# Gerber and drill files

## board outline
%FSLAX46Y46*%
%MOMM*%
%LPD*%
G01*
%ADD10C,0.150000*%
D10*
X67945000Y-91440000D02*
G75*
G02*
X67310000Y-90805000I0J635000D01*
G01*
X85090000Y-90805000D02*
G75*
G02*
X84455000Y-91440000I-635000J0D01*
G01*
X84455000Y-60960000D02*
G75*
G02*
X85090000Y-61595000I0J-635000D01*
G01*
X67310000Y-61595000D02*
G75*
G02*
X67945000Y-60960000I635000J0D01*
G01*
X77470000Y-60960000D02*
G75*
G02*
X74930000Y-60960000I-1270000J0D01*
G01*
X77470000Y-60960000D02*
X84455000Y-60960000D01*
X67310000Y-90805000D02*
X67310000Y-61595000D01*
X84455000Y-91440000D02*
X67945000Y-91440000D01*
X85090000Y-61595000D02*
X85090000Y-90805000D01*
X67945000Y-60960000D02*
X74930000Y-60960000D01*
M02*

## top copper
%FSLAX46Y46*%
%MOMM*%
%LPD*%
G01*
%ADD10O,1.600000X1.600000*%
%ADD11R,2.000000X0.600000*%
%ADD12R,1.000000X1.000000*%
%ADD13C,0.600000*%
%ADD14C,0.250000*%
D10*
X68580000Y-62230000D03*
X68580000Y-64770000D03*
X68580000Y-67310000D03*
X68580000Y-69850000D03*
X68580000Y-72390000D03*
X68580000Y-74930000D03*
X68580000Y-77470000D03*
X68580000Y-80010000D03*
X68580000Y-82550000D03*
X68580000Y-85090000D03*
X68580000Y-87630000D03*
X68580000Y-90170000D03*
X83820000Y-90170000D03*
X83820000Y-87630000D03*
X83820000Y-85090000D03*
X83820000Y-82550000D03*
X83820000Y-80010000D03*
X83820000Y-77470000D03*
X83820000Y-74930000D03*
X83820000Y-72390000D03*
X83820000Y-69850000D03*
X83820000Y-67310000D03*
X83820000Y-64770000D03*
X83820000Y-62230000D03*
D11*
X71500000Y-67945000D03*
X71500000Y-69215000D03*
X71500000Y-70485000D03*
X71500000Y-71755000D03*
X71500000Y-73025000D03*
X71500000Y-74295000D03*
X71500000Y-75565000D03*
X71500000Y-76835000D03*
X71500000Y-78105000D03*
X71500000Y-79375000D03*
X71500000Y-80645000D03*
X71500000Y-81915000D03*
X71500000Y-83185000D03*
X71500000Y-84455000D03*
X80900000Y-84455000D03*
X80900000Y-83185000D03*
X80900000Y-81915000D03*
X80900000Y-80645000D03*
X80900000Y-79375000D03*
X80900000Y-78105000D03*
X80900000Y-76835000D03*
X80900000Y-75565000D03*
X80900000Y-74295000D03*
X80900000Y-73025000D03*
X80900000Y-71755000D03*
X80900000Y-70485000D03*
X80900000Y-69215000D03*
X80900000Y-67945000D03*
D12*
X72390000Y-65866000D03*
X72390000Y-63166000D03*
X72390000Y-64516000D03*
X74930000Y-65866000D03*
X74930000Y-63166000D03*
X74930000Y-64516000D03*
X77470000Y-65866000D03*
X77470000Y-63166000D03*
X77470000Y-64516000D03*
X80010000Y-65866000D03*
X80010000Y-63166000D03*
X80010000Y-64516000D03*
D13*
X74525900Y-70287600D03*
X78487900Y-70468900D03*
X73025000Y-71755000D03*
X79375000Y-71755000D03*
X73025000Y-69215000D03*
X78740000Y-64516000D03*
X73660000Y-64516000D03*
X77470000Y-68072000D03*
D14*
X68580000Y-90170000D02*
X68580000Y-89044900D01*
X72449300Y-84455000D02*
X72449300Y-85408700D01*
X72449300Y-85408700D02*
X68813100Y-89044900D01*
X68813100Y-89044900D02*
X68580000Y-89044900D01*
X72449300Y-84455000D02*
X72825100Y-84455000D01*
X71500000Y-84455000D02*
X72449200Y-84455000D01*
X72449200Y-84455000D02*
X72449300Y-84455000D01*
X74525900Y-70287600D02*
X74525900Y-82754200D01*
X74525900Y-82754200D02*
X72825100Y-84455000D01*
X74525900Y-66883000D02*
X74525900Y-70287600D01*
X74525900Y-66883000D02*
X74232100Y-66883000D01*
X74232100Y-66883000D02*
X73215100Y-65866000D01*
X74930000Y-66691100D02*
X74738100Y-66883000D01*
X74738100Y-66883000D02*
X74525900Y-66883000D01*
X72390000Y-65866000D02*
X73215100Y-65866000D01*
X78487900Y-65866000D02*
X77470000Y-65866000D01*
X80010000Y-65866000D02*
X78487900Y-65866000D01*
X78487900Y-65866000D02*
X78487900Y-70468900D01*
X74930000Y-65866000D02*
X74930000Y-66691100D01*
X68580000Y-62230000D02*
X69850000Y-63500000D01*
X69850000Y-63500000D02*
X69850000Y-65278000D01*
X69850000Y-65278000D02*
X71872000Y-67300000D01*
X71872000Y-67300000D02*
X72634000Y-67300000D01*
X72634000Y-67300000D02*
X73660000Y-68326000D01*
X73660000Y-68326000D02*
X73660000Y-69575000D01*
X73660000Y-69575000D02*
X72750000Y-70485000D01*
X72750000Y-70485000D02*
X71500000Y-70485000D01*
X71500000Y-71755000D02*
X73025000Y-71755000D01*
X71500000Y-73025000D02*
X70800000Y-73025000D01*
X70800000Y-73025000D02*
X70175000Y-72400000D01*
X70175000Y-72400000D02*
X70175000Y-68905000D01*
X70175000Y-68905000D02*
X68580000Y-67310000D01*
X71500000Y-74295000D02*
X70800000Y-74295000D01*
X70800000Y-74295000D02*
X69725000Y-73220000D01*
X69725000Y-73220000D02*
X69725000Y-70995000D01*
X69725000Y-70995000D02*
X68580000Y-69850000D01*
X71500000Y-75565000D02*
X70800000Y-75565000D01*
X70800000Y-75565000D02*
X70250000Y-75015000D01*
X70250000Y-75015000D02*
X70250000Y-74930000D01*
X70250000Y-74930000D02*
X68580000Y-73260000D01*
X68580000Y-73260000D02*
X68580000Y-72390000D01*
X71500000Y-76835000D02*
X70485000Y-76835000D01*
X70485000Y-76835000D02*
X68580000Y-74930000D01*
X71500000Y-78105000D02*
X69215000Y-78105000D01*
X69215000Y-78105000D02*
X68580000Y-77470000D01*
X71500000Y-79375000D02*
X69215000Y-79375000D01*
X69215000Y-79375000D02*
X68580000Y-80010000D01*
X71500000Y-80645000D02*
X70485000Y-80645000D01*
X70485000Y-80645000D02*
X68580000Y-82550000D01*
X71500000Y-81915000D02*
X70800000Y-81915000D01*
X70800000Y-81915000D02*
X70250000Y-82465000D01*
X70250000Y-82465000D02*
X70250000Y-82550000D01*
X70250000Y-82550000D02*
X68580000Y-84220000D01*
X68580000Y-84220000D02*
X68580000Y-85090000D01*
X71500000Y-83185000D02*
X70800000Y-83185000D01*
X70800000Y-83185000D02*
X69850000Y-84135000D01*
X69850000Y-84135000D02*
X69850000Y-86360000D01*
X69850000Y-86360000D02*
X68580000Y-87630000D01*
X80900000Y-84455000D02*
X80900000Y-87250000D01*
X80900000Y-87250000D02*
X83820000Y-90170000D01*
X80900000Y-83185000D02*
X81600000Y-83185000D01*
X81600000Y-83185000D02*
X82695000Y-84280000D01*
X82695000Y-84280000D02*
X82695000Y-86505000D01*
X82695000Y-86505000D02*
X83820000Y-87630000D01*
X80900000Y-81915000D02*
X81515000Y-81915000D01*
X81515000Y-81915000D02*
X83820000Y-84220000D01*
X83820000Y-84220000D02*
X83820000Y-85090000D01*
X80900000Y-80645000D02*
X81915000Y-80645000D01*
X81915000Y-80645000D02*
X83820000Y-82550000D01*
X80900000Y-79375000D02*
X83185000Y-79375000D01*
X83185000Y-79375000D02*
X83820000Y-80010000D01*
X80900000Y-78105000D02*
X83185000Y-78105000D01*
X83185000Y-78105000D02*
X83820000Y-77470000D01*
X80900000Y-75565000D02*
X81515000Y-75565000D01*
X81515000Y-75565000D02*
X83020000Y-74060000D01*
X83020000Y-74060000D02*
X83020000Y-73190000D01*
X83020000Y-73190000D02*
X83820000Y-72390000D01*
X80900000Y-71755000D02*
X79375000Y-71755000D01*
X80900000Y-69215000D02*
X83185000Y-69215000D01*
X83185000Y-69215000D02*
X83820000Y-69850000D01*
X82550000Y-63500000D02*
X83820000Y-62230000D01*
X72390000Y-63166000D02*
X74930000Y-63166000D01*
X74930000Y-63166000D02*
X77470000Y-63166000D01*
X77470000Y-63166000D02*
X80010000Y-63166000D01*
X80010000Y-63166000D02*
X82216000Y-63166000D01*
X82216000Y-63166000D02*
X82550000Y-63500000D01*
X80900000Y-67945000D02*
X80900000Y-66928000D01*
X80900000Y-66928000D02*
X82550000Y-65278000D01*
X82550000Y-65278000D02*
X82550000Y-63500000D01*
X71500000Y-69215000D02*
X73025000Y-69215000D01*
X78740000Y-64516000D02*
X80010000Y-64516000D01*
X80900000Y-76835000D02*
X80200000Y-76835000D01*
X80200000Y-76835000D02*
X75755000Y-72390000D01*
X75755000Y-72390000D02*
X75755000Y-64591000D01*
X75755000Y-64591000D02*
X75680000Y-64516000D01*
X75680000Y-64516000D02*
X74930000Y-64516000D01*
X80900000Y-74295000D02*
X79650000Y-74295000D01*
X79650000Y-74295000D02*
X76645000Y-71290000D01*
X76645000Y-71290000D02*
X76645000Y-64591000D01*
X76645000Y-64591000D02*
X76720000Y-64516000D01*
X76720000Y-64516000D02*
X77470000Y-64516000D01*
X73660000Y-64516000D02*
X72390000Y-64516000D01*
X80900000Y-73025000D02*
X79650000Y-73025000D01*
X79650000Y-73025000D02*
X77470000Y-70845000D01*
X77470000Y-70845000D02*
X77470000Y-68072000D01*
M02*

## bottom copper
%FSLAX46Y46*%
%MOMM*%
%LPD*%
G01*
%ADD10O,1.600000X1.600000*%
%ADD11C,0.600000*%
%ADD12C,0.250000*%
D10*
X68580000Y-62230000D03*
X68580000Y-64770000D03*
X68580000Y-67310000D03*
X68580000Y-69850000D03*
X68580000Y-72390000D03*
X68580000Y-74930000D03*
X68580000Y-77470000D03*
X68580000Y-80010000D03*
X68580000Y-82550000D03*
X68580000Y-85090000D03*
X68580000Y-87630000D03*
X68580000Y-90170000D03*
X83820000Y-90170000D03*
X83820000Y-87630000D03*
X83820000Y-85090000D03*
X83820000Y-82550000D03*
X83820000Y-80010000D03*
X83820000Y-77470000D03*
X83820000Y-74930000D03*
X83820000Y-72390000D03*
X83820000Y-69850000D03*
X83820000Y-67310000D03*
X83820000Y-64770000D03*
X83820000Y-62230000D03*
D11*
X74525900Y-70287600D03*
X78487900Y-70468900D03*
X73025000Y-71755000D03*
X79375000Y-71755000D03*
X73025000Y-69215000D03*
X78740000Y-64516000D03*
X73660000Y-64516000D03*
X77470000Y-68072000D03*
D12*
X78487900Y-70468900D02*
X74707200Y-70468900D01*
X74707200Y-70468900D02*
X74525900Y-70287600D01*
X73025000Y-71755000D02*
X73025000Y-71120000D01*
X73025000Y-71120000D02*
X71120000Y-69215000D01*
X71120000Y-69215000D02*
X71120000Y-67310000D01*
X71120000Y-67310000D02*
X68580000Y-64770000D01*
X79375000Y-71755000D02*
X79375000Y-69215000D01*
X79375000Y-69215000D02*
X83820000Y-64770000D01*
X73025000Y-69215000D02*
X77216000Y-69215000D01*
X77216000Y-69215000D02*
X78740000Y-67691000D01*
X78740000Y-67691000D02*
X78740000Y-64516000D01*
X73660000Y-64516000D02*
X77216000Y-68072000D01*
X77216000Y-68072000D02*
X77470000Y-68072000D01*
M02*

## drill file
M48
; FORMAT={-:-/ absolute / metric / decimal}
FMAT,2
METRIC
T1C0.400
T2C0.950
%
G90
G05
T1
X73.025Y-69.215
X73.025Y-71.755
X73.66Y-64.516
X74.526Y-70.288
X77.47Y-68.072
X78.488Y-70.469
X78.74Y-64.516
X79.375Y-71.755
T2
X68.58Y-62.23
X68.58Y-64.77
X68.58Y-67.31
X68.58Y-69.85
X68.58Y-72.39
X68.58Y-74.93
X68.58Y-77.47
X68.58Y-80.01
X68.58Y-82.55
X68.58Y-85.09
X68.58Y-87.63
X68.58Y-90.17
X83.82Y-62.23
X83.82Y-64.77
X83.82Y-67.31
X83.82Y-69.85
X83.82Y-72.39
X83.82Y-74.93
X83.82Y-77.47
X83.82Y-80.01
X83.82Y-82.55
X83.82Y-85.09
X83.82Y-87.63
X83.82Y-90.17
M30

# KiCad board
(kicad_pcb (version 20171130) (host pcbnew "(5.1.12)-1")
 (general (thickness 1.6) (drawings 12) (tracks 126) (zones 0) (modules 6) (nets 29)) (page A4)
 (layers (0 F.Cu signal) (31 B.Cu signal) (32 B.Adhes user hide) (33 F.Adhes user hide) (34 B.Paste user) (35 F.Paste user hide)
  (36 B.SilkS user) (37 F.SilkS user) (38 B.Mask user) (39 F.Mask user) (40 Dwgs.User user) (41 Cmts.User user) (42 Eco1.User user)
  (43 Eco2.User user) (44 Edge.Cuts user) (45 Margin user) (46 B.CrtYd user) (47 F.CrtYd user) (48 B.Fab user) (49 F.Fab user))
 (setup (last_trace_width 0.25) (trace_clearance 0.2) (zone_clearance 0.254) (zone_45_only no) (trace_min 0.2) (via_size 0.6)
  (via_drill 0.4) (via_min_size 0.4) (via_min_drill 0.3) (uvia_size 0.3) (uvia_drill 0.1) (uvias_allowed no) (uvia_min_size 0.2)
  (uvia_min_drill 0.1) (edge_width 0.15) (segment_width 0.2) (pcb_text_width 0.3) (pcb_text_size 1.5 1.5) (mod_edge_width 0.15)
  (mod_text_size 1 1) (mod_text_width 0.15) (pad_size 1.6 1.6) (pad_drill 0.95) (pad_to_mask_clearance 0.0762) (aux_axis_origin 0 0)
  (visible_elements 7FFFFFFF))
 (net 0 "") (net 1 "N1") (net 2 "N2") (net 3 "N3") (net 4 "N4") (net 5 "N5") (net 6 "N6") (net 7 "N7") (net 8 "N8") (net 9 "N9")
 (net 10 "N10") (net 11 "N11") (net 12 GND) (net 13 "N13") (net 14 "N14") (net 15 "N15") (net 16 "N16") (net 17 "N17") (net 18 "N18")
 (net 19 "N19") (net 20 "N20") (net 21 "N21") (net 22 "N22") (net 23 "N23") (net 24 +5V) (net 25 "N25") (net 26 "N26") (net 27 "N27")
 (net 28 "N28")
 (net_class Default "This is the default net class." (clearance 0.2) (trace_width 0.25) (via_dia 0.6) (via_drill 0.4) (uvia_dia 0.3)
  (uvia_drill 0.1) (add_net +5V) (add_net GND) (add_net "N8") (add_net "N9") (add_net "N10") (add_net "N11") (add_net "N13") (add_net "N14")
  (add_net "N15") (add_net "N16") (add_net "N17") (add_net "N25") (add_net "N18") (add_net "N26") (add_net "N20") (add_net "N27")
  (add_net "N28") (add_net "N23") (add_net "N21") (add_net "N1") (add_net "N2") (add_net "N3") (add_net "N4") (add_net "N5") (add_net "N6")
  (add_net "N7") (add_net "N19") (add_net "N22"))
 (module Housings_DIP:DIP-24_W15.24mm (layer F.Cu) (at 68.58 62.23)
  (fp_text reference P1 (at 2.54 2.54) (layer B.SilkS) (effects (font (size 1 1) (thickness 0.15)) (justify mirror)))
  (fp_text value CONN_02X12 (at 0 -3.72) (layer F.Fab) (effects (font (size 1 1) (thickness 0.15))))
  (pad 1 thru_hole oval (at 0 0) (size 1.6 1.6) (drill 0.95) (layers *.Cu *.Mask F.SilkS) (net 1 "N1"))
  (pad 2 thru_hole oval (at 0 2.54) (size 1.6 1.6) (drill 0.95) (layers *.Cu *.Mask F.SilkS) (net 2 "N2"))
  (pad 3 thru_hole oval (at 0 5.08) (size 1.6 1.6) (drill 0.95) (layers *.Cu *.Mask F.SilkS) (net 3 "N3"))
  (pad 4 thru_hole oval (at 0 7.62) (size 1.6 1.6) (drill 0.95) (layers *.Cu *.Mask F.SilkS) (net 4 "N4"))
  (pad 5 thru_hole oval (at 0 10.16) (size 1.6 1.6) (drill 0.95) (layers *.Cu *.Mask F.SilkS) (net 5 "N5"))
  (pad 6 thru_hole oval (at 0 12.7) (size 1.6 1.6) (drill 0.95) (layers *.Cu *.Mask F.SilkS) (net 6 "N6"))
  (pad 7 thru_hole oval (at 0 15.24) (size 1.6 1.6) (drill 0.95) (layers *.Cu *.Mask F.SilkS) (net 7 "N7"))
  (pad 8 thru_hole oval (at 0 17.78) (size 1.6 1.6) (drill 0.95) (layers *.Cu *.Mask F.SilkS) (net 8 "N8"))
  (pad 9 thru_hole oval (at 0 20.32) (size 1.6 1.6) (drill 0.95) (layers *.Cu *.Mask F.SilkS) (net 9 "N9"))
  (pad 10 thru_hole oval (at 0 22.86) (size 1.6 1.6) (drill 0.95) (layers *.Cu *.Mask F.SilkS) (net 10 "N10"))
  (pad 11 thru_hole oval (at 0 25.4) (size 1.6 1.6) (drill 0.95) (layers *.Cu *.Mask F.SilkS) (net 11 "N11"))
  (pad 12 thru_hole oval (at 0 27.94) (size 1.6 1.6) (drill 0.95) (layers *.Cu *.Mask F.SilkS) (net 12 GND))
  (pad 13 thru_hole oval (at 15.24 27.94) (size 1.6 1.6) (drill 0.95) (layers *.Cu *.Mask F.SilkS) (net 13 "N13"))
  (pad 14 thru_hole oval (at 15.24 25.4) (size 1.6 1.6) (drill 0.95) (layers *.Cu *.Mask F.SilkS) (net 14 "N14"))
  (pad 15 thru_hole oval (at 15.24 22.86) (size 1.6 1.6) (drill 0.95) (layers *.Cu *.Mask F.SilkS) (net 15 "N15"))
  (pad 16 thru_hole oval (at 15.24 20.32) (size 1.6 1.6) (drill 0.95) (layers *.Cu *.Mask F.SilkS) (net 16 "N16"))
  (pad 17 thru_hole oval (at 15.24 17.78) (size 1.6 1.6) (drill 0.95) (layers *.Cu *.Mask F.SilkS) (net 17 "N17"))
  (pad 18 thru_hole oval (at 15.24 15.24) (size 1.6 1.6) (drill 0.95) (layers *.Cu *.Mask F.SilkS) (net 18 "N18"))
  (pad 19 thru_hole oval (at 15.24 12.7) (size 1.6 1.6) (drill 0.95) (layers *.Cu *.Mask F.SilkS) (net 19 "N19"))
  (pad 20 thru_hole oval (at 15.24 10.16) (size 1.6 1.6) (drill 0.95) (layers *.Cu *.Mask F.SilkS) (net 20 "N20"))
  (pad 21 thru_hole oval (at 15.24 7.62) (size 1.6 1.6) (drill 0.95) (layers *.Cu *.Mask F.SilkS) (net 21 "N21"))
  (pad 22 thru_hole oval (at 15.24 5.08) (size 1.6 1.6) (drill 0.95) (layers *.Cu *.Mask F.SilkS) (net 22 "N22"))
  (pad 23 thru_hole oval (at 15.24 2.54) (size 1.6 1.6) (drill 0.95) (layers *.Cu *.Mask F.SilkS) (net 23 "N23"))
  (pad 24 thru_hole oval (at 15.24 0) (size 1.6 1.6) (drill 0.95) (layers *.Cu *.Mask F.SilkS) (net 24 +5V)))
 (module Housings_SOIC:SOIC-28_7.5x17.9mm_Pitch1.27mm (layer F.Cu) (at 76.2 76.2)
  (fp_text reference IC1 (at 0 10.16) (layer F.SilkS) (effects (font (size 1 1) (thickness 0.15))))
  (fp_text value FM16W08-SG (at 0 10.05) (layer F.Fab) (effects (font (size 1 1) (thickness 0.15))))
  (pad 1 smd rect (at -4.7 -8.255) (size 2 0.6) (layers F.Cu F.Paste F.Mask))
  (pad 2 smd rect (at -4.7 -6.985) (size 2 0.6) (layers F.Cu F.Paste F.Mask) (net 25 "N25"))
  (pad 3 smd rect (at -4.7 -5.715) (size 2 0.6) (layers F.Cu F.Paste F.Mask) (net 1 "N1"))
  (pad 4 smd rect (at -4.7 -4.445) (size 2 0.6) (layers F.Cu F.Paste F.Mask) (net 2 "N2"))
  (pad 5 smd rect (at -4.7 -3.175) (size 2 0.6) (layers F.Cu F.Paste F.Mask) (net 3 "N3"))
  (pad 6 smd rect (at -4.7 -1.905) (size 2 0.6) (layers F.Cu F.Paste F.Mask) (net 4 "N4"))
  (pad 7 smd rect (at -4.7 -0.635) (size 2 0.6) (layers F.Cu F.Paste F.Mask) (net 5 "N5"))
  (pad 8 smd rect (at -4.7 0.635) (size 2 0.6) (layers F.Cu F.Paste F.Mask) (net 6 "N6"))
  (pad 9 smd rect (at -4.7 1.905) (size 2 0.6) (layers F.Cu F.Paste F.Mask) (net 7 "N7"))
  (pad 10 smd rect (at -4.7 3.175) (size 2 0.6) (layers F.Cu F.Paste F.Mask) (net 8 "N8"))
  (pad 11 smd rect (at -4.7 4.445) (size 2 0.6) (layers F.Cu F.Paste F.Mask) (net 9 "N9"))
  (pad 12 smd rect (at -4.7 5.715) (size 2 0.6) (layers F.Cu F.Paste F.Mask) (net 10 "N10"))
  (pad 13 smd rect (at -4.7 6.985) (size 2 0.6) (layers F.Cu F.Paste F.Mask) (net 11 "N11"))
  (pad 14 smd rect (at -4.7 8.255) (size 2 0.6) (layers F.Cu F.Paste F.Mask) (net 12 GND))
  (pad 15 smd rect (at 4.7 8.255) (size 2 0.6) (layers F.Cu F.Paste F.Mask) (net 13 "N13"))
  (pad 16 smd rect (at 4.7 6.985) (size 2 0.6) (layers F.Cu F.Paste F.Mask) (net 14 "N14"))
  (pad 17 smd rect (at 4.7 5.715) (size 2 0.6) (layers F.Cu F.Paste F.Mask) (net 15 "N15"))
  (pad 18 smd rect (at 4.7 4.445) (size 2 0.6) (layers F.Cu F.Paste F.Mask) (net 16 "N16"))
  (pad 19 smd rect (at 4.7 3.175) (size 2 0.6) (layers F.Cu F.Paste F.Mask) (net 17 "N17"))
  (pad 20 smd rect (at 4.7 1.905) (size 2 0.6) (layers F.Cu F.Paste F.Mask) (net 18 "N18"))
  (pad 21 smd rect (at 4.7 0.635) (size 2 0.6) (layers F.Cu F.Paste F.Mask) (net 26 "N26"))
  (pad 22 smd rect (at 4.7 -0.635) (size 2 0.6) (layers F.Cu F.Paste F.Mask) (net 20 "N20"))
  (pad 23 smd rect (at 4.7 -1.905) (size 2 0.6) (layers F.Cu F.Paste F.Mask) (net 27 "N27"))
  (pad 24 smd rect (at 4.7 -3.175) (size 2 0.6) (layers F.Cu F.Paste F.Mask) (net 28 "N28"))
  (pad 25 smd rect (at 4.7 -4.445) (size 2 0.6) (layers F.Cu F.Paste F.Mask) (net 23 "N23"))
  (pad 26 smd rect (at 4.7 -5.715) (size 2 0.6) (layers F.Cu F.Paste F.Mask))
  (pad 27 smd rect (at 4.7 -6.985) (size 2 0.6) (layers F.Cu F.Paste F.Mask) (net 21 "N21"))
  (pad 28 smd rect (at 4.7 -8.255) (size 2 0.6) (layers F.Cu F.Paste F.Mask) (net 24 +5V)))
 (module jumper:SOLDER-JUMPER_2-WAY (layer F.Cu) (at 72.39 64.516 90)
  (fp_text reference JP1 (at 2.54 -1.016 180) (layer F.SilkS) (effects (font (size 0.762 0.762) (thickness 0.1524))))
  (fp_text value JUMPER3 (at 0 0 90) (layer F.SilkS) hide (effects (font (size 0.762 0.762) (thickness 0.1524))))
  (pad 1 smd rect (at -1.35 0 90) (size 1 1) (layers F.Cu F.Paste F.Mask) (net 12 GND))
  (pad 3 smd rect (at 1.35 0 90) (size 1 1) (layers F.Cu F.Paste F.Mask) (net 24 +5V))
  (pad 2 smd rect (at 0 0 90) (size 1 1) (layers F.Cu F.Paste F.Mask) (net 28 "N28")))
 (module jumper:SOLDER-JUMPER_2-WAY (layer F.Cu) (at 74.93 64.516 90)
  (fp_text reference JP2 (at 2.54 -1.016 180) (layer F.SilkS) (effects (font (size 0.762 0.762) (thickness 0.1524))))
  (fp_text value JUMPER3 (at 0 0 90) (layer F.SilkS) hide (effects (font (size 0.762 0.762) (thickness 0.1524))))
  (pad 1 smd rect (at -1.35 0 90) (size 1 1) (layers F.Cu F.Paste F.Mask) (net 12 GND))
  (pad 3 smd rect (at 1.35 0 90) (size 1 1) (layers F.Cu F.Paste F.Mask) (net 24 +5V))
  (pad 2 smd rect (at 0 0 90) (size 1 1) (layers F.Cu F.Paste F.Mask) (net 26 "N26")))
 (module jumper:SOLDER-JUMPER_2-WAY (layer F.Cu) (at 77.47 64.516 90)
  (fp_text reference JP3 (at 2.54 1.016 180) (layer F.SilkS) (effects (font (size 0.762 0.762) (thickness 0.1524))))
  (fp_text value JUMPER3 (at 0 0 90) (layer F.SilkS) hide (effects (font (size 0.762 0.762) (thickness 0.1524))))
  (pad 1 smd rect (at -1.35 0 90) (size 1 1) (layers F.Cu F.Paste F.Mask) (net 12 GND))
  (pad 3 smd rect (at 1.35 0 90) (size 1 1) (layers F.Cu F.Paste F.Mask) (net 24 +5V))
  (pad 2 smd rect (at 0 0 90) (size 1 1) (layers F.Cu F.Paste F.Mask) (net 27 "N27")))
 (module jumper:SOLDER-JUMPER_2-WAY (layer F.Cu) (at 80.01 64.516 90)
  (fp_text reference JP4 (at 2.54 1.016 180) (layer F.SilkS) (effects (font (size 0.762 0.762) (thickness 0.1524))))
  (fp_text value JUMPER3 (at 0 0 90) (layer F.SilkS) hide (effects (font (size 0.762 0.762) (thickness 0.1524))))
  (pad 1 smd rect (at -1.35 0 90) (size 1 1) (layers F.Cu F.Paste F.Mask) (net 12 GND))
  (pad 3 smd rect (at 1.35 0 90) (size 1 1) (layers F.Cu F.Paste F.Mask) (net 24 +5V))
  (pad 2 smd rect (at 0 0 90) (size 1 1) (layers F.Cu F.Paste F.Mask) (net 25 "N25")))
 (gr_arc (start 67.945 90.805) (end 67.945 91.44) (angle 90) (layer Edge.Cuts) (width 0.15))
 (gr_arc (start 84.455 90.805) (end 85.09 90.805) (angle 90) (layer Edge.Cuts) (width 0.15))
 (gr_arc (start 84.455 61.595) (end 84.455 60.96) (angle 90) (layer Edge.Cuts) (width 0.15))
 (gr_arc (start 67.945 61.595) (end 67.31 61.595) (angle 90) (layer Edge.Cuts) (width 0.15))
 (gr_arc (start 76.2 60.96) (end 77.47 60.96) (angle 180) (layer Edge.Cuts) (width 0.15))
 (gr_line (start 77.47 60.96) (end 84.455 60.96) (layer Edge.Cuts) (width 0.15))
 (gr_line (start 67.31 90.805) (end 67.31 61.595) (layer Edge.Cuts) (width 0.15))
 (gr_line (start 84.455 91.44) (end 67.945 91.44) (layer Edge.Cuts) (width 0.15))
 (gr_line (start 85.09 61.595) (end 85.09 90.805) (layer Edge.Cuts) (width 0.15))
 (gr_line (start 67.945 60.96) (end 74.93 60.96) (layer Edge.Cuts) (width 0.15))
 (segment (start 68.58 90.17) (end 68.58 89.0449) (width 0.25) (layer F.Cu) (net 12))
 (segment (start 72.4493 84.455) (end 72.4493 85.4087) (width 0.25) (layer F.Cu) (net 12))
 (segment (start 72.4493 85.4087) (end 68.8131 89.0449) (width 0.25) (layer F.Cu) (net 12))
 (segment (start 68.8131 89.0449) (end 68.58 89.0449) (width 0.25) (layer F.Cu) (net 12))
 (segment (start 72.4493 84.455) (end 72.8251 84.455) (width 0.25) (layer F.Cu) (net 12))
 (segment (start 71.5 84.455) (end 72.4492 84.455) (width 0.25) (layer F.Cu) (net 12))
 (segment (start 72.4492 84.455) (end 72.4493 84.455) (width 0.25) (layer F.Cu) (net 12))
 (segment (start 74.5259 70.2876) (end 74.5259 82.7542) (width 0.25) (layer F.Cu) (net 12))
 (segment (start 74.5259 82.7542) (end 72.8251 84.455) (width 0.25) (layer F.Cu) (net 12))
 (segment (start 74.5259 66.883) (end 74.5259 70.2876) (width 0.25) (layer F.Cu) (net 12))
 (segment (start 74.5259 66.883) (end 74.2321 66.883) (width 0.25) (layer F.Cu) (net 12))
 (segment (start 74.2321 66.883) (end 73.2151 65.866) (width 0.25) (layer F.Cu) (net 12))
 (segment (start 74.93 66.6911) (end 74.7381 66.883) (width 0.25) (layer F.Cu) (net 12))
 (segment (start 74.7381 66.883) (end 74.5259 66.883) (width 0.25) (layer F.Cu) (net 12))
 (segment (start 72.39 65.866) (end 73.2151 65.866) (width 0.25) (layer F.Cu) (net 12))
 (segment (start 78.4879 65.866) (end 77.47 65.866) (width 0.25) (layer F.Cu) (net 12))
 (segment (start 80.01 65.866) (end 78.4879 65.866) (width 0.25) (layer F.Cu) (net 12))
 (segment (start 78.4879 65.866) (end 78.4879 70.4689) (width 0.25) (layer F.Cu) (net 12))
 (segment (start 78.4879 70.4689) (end 74.7072 70.4689) (width 0.25) (layer B.Cu) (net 12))
 (segment (start 74.7072 70.4689) (end 74.5259 70.2876) (width 0.25) (layer B.Cu) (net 12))
 (segment (start 74.93 65.866) (end 74.93 66.6911) (width 0.25) (layer F.Cu) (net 12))
 (via (at 74.5259 70.2876) (size 0.6) (layers F.Cu B.Cu) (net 12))
 (via (at 78.4879 70.4689) (size 0.6) (layers F.Cu B.Cu) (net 12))
 (segment (start 68.58 62.23) (end 69.85 63.5) (width 0.25) (layer F.Cu) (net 1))
 (segment (start 69.85 63.5) (end 69.85 65.278) (width 0.25) (layer F.Cu) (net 1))
 (segment (start 69.85 65.278) (end 71.872 67.3) (width 0.25) (layer F.Cu) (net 1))
 (segment (start 71.872 67.3) (end 72.634 67.3) (width 0.25) (layer F.Cu) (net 1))
 (segment (start 72.634 67.3) (end 73.66 68.326) (width 0.25) (layer F.Cu) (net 1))
 (segment (start 73.66 68.326) (end 73.66 69.575) (width 0.25) (layer F.Cu) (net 1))
 (segment (start 73.66 69.575) (end 72.75 70.485) (width 0.25) (layer F.Cu) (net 1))
 (segment (start 72.75 70.485) (end 71.5 70.485) (width 0.25) (layer F.Cu) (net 1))
 (segment (start 71.5 71.755) (end 73.025 71.755) (width 0.25) (layer F.Cu) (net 2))
 (segment (start 73.025 71.755) (end 73.025 71.12) (width 0.25) (layer B.Cu) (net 2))
 (segment (start 73.025 71.12) (end 71.12 69.215) (width 0.25) (layer B.Cu) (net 2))
 (segment (start 71.12 69.215) (end 71.12 67.31) (width 0.25) (layer B.Cu) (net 2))
 (segment (start 71.12 67.31) (end 68.58 64.77) (width 0.25) (layer B.Cu) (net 2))
 (via (at 73.025 71.755) (size 0.6) (layers F.Cu B.Cu) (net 2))
 (segment (start 71.5 73.025) (end 70.8 73.025) (width 0.25) (layer F.Cu) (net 3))
 (segment (start 70.8 73.025) (end 70.175 72.4) (width 0.25) (layer F.Cu) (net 3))
 (segment (start 70.175 72.4) (end 70.175 68.905) (width 0.25) (layer F.Cu) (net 3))
 (segment (start 70.175 68.905) (end 68.58 67.31) (width 0.25) (layer F.Cu) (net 3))
 (segment (start 71.5 74.295) (end 70.8 74.295) (width 0.25) (layer F.Cu) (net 4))
 (segment (start 70.8 74.295) (end 69.725 73.22) (width 0.25) (layer F.Cu) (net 4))
 (segment (start 69.725 73.22) (end 69.725 70.995) (width 0.25) (layer F.Cu) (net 4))
 (segment (start 69.725 70.995) (end 68.58 69.85) (width 0.25) (layer F.Cu) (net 4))
 (segment (start 71.5 75.565) (end 70.8 75.565) (width 0.25) (layer F.Cu) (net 5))
 (segment (start 70.8 75.565) (end 70.25 75.015) (width 0.25) (layer F.Cu) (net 5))
 (segment (start 70.25 75.015) (end 70.25 74.93) (width 0.25) (layer F.Cu) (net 5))
 (segment (start 70.25 74.93) (end 68.58 73.26) (width 0.25) (layer F.Cu) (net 5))
 (segment (start 68.58 73.26) (end 68.58 72.39) (width 0.25) (layer F.Cu) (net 5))
 (segment (start 71.5 76.835) (end 70.485 76.835) (width 0.25) (layer F.Cu) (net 6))
 (segment (start 70.485 76.835) (end 68.58 74.93) (width 0.25) (layer F.Cu) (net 6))
 (segment (start 71.5 78.105) (end 69.215 78.105) (width 0.25) (layer F.Cu) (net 7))
 (segment (start 69.215 78.105) (end 68.58 77.47) (width 0.25) (layer F.Cu) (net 7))
 (segment (start 71.5 79.375) (end 69.215 79.375) (width 0.25) (layer F.Cu) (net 8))
 (segment (start 69.215 79.375) (end 68.58 80.01) (width 0.25) (layer F.Cu) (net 8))
 (segment (start 71.5 80.645) (end 70.485 80.645) (width 0.25) (layer F.Cu) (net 9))
 (segment (start 70.485 80.645) (end 68.58 82.55) (width 0.25) (layer F.Cu) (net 9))
 (segment (start 71.5 81.915) (end 70.8 81.915) (width 0.25) (layer F.Cu) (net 10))
 (segment (start 70.8 81.915) (end 70.25 82.465) (width 0.25) (layer F.Cu) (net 10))
 (segment (start 70.25 82.465) (end 70.25 82.55) (width 0.25) (layer F.Cu) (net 10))
 (segment (start 70.25 82.55) (end 68.58 84.22) (width 0.25) (layer F.Cu) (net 10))
 (segment (start 68.58 84.22) (end 68.58 85.09) (width 0.25) (layer F.Cu) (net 10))
 (segment (start 71.5 83.185) (end 70.8 83.185) (width 0.25) (layer F.Cu) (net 11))
 (segment (start 70.8 83.185) (end 69.85 84.135) (width 0.25) (layer F.Cu) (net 11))
 (segment (start 69.85 84.135) (end 69.85 86.36) (width 0.25) (layer F.Cu) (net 11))
 (segment (start 69.85 86.36) (end 68.58 87.63) (width 0.25) (layer F.Cu) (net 11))
 (segment (start 80.9 84.455) (end 80.9 87.25) (width 0.25) (layer F.Cu) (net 13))
 (segment (start 80.9 87.25) (end 83.82 90.17) (width 0.25) (layer F.Cu) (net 13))
 (segment (start 80.9 83.185) (end 81.6 83.185) (width 0.25) (layer F.Cu) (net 14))
 (segment (start 81.6 83.185) (end 82.695 84.28) (width 0.25) (layer F.Cu) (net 14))
 (segment (start 82.695 84.28) (end 82.695 86.505) (width 0.25) (layer F.Cu) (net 14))
 (segment (start 82.695 86.505) (end 83.82 87.63) (width 0.25) (layer F.Cu) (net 14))
 (segment (start 80.9 81.915) (end 81.515 81.915) (width 0.25) (layer F.Cu) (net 15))
 (segment (start 81.515 81.915) (end 83.82 84.22) (width 0.25) (layer F.Cu) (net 15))
 (segment (start 83.82 84.22) (end 83.82 85.09) (width 0.25) (layer F.Cu) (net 15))
 (segment (start 80.9 80.645) (end 81.915 80.645) (width 0.25) (layer F.Cu) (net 16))
 (segment (start 81.915 80.645) (end 83.82 82.55) (width 0.25) (layer F.Cu) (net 16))
 (segment (start 80.9 79.375) (end 83.185 79.375) (width 0.25) (layer F.Cu) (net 17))
 (segment (start 83.185 79.375) (end 83.82 80.01) (width 0.25) (layer F.Cu) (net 17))
 (segment (start 80.9 78.105) (end 83.185 78.105) (width 0.25) (layer F.Cu) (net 18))
 (segment (start 83.185 78.105) (end 83.82 77.47) (width 0.25) (layer F.Cu) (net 18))
 (segment (start 80.9 75.565) (end 81.515 75.565) (width 0.25) (layer F.Cu) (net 20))
 (segment (start 81.515 75.565) (end 83.02 74.06) (width 0.25) (layer F.Cu) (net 20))
 (segment (start 83.02 74.06) (end 83.02 73.19) (width 0.25) (layer F.Cu) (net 20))
 (segment (start 83.02 73.19) (end 83.82 72.39) (width 0.25) (layer F.Cu) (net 20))
 (segment (start 80.9 71.755) (end 79.375 71.755) (width 0.25) (layer F.Cu) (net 23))
 (segment (start 79.375 71.755) (end 79.375 69.215) (width 0.25) (layer B.Cu) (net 23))
 (segment (start 79.375 69.215) (end 83.82 64.77) (width 0.25) (layer B.Cu) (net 23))
 (via (at 79.375 71.755) (size 0.6) (layers F.Cu B.Cu) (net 23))
 (segment (start 80.9 69.215) (end 83.185 69.215) (width 0.25) (layer F.Cu) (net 21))
 (segment (start 83.185 69.215) (end 83.82 69.85) (width 0.25) (layer F.Cu) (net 21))
 (segment (start 82.55 63.5) (end 83.82 62.23) (width 0.25) (layer F.Cu) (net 24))
 (segment (start 72.39 63.166) (end 74.93 63.166) (width 0.25) (layer F.Cu) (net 24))
 (segment (start 74.93 63.166) (end 77.47 63.166) (width 0.25) (layer F.Cu) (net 24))
 (segment (start 77.47 63.166) (end 80.01 63.166) (width 0.25) (layer F.Cu) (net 24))
 (segment (start 80.01 63.166) (end 82.216 63.166) (width 0.25) (layer F.Cu) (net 24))
 (segment (start 82.216 63.166) (end 82.55 63.5) (width 0.25) (layer F.Cu) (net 24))
 (segment (start 80.9 67.945) (end 80.9 66.928) (width 0.25) (layer F.Cu) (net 24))
 (segment (start 80.9 66.928) (end 82.55 65.278) (width 0.25) (layer F.Cu) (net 24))
 (segment (start 82.55 65.278) (end 82.55 63.5) (width 0.25) (layer F.Cu) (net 24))
 (segment (start 71.5 69.215) (end 73.025 69.215) (width 0.25) (layer F.Cu) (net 25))
 (segment (start 78.74 64.516) (end 80.01 64.516) (width 0.25) (layer F.Cu) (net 25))
 (segment (start 73.025 69.215) (end 77.216 69.215) (width 0.25) (layer B.Cu) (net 25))
 (segment (start 77.216 69.215) (end 78.74 67.691) (width 0.25) (layer B.Cu) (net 25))
 (segment (start 78.74 67.691) (end 78.74 64.516) (width 0.25) (layer B.Cu) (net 25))
 (via (at 73.025 69.215) (size 0.6) (layers F.Cu B.Cu) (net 25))
 (via (at 78.74 64.516) (size 0.6) (layers F.Cu B.Cu) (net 25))
 (segment (start 80.9 76.835) (end 80.2 76.835) (width 0.25) (layer F.Cu) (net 26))
 (segment (start 80.2 76.835) (end 75.755 72.39) (width 0.25) (layer F.Cu) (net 26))
 (segment (start 75.755 72.39) (end 75.755 64.591) (width 0.25) (layer F.Cu) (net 26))
 (segment (start 75.755 64.591) (end 75.68 64.516) (width 0.25) (layer F.Cu) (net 26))
 (segment (start 75.68 64.516) (end 74.93 64.516) (width 0.25) (layer F.Cu) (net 26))
 (segment (start 80.9 74.295) (end 79.65 74.295) (width 0.25) (layer F.Cu) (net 27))
 (segment (start 79.65 74.295) (end 76.645 71.29) (width 0.25) (layer F.Cu) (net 27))
 (segment (start 76.645 71.29) (end 76.645 64.591) (width 0.25) (layer F.Cu) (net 27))
 (segment (start 76.645 64.591) (end 76.72 64.516) (width 0.25) (layer F.Cu) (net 27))
 (segment (start 76.72 64.516) (end 77.47 64.516) (width 0.25) (layer F.Cu) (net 27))
 (segment (start 73.66 64.516) (end 72.39 64.516) (width 0.25) (layer F.Cu) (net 28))
 (segment (start 73.66 64.516) (end 77.216 68.072) (width 0.25) (layer B.Cu) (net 28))
 (segment (start 77.216 68.072) (end 77.47 68.072) (width 0.25) (layer B.Cu) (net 28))
 (segment (start 80.9 73.025) (end 79.65 73.025) (width 0.25) (layer F.Cu) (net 28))
 (segment (start 79.65 73.025) (end 77.47 70.845) (width 0.25) (layer F.Cu) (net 28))
 (segment (start 77.47 70.845) (end 77.47 68.072) (width 0.25) (layer F.Cu) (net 28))
 (via (at 73.66 64.516) (size 0.6) (layers F.Cu B.Cu) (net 28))
 (via (at 77.47 68.072) (size 0.6) (layers F.Cu B.Cu) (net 28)))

